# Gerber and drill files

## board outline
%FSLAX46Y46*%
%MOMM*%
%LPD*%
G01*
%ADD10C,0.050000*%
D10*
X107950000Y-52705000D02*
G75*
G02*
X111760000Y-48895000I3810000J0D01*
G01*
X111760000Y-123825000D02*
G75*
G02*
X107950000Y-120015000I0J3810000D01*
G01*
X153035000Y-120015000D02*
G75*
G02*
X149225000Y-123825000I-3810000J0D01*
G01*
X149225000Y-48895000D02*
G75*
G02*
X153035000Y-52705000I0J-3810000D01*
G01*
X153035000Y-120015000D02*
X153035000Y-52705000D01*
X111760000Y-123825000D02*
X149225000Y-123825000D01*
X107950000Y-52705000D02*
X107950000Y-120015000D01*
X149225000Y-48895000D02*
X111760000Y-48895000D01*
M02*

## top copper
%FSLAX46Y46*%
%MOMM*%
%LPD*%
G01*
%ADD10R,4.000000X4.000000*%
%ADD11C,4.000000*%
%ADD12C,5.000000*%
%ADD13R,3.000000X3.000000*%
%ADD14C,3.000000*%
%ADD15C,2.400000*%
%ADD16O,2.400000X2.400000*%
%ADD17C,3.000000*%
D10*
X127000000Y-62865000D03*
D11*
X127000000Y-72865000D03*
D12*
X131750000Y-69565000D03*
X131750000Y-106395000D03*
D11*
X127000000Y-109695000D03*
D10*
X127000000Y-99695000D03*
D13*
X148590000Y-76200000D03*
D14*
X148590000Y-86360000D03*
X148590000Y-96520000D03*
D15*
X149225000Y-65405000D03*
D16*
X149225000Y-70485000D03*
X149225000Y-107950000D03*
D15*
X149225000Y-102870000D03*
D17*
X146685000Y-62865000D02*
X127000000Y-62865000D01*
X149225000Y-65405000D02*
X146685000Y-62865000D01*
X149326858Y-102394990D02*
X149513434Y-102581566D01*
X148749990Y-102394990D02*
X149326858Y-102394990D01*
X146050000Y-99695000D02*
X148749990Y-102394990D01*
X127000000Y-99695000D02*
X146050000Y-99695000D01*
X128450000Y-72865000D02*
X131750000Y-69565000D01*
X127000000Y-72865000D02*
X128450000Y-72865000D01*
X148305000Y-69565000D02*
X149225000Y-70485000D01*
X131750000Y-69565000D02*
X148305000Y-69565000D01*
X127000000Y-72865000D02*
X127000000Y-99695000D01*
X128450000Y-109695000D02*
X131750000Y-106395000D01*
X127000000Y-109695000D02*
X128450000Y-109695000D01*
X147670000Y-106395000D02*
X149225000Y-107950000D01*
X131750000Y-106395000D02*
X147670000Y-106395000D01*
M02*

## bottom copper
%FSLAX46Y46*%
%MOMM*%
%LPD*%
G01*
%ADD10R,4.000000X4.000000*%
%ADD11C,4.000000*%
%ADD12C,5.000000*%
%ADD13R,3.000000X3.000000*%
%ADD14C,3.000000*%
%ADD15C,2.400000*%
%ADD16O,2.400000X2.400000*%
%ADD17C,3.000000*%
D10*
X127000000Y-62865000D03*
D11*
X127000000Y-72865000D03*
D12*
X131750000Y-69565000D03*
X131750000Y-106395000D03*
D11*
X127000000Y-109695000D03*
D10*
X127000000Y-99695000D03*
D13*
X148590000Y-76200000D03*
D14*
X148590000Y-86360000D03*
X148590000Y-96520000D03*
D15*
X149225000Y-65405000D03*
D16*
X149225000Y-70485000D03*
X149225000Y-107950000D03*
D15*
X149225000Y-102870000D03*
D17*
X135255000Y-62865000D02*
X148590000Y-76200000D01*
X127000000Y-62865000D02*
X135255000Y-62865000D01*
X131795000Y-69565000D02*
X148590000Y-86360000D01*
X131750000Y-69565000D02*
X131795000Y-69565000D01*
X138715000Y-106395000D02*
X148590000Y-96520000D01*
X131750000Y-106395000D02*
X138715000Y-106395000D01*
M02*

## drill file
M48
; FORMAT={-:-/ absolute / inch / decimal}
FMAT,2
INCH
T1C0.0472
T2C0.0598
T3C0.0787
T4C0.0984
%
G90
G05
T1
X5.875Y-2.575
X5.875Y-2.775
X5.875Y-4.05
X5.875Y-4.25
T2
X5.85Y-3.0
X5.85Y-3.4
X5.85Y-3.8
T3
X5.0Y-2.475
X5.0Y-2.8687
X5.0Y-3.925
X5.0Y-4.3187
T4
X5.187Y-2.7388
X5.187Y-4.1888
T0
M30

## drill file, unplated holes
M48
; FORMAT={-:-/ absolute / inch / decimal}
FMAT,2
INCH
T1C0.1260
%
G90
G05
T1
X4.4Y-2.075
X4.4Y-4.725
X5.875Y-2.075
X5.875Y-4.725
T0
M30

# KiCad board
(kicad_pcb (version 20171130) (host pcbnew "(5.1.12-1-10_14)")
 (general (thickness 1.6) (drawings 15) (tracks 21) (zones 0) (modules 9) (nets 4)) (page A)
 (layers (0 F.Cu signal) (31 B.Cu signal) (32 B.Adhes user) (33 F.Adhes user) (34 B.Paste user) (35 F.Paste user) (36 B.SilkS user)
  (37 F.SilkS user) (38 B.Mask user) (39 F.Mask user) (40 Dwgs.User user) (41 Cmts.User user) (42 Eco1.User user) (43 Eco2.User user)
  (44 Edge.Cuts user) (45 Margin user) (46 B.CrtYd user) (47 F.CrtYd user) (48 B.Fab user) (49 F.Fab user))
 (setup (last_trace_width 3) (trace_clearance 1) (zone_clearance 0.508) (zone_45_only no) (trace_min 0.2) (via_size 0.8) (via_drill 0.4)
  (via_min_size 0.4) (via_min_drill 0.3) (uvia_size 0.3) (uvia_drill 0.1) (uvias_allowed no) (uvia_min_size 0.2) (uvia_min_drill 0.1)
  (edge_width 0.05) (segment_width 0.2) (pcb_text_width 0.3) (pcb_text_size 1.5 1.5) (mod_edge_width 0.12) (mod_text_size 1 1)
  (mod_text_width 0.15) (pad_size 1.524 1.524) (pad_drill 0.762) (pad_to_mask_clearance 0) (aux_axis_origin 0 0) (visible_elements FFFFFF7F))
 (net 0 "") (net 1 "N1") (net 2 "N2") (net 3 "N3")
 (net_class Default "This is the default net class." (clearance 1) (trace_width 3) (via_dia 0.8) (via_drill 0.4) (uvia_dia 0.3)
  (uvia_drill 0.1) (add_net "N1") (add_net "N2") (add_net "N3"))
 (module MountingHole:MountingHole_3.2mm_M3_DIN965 (layer F.Cu) (at 111.76 52.705)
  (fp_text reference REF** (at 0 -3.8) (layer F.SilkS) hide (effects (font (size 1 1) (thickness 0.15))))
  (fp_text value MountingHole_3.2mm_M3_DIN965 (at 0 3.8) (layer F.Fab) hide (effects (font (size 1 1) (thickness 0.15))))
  (pad 1 np_thru_hole circle (at 0 0) (size 3.2 3.2) (drill 3.2) (layers *.Cu *.Mask)))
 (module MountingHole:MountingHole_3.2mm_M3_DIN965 (layer F.Cu) (at 111.76 120.015)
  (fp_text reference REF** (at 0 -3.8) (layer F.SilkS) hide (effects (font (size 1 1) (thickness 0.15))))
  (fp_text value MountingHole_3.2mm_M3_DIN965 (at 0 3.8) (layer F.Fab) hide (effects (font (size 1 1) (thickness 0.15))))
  (pad 1 np_thru_hole circle (at 0 0) (size 3.2 3.2) (drill 3.2) (layers *.Cu *.Mask)))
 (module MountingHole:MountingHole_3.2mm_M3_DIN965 (layer F.Cu) (at 149.225 120.015)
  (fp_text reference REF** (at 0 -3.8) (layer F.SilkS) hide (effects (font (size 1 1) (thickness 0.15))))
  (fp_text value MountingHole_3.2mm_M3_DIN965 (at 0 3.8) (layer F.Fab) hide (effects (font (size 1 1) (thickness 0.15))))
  (pad 1 np_thru_hole circle (at 0 0) (size 3.2 3.2) (drill 3.2) (layers *.Cu *.Mask)))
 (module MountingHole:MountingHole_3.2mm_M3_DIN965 (layer F.Cu) (at 149.225 52.705)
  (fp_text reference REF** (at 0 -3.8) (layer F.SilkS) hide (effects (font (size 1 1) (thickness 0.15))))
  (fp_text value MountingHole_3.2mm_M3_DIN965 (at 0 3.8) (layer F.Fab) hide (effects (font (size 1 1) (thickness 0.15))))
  (pad 1 np_thru_hole circle (at 0 0) (size 3.2 3.2) (drill 3.2) (layers *.Cu *.Mask)))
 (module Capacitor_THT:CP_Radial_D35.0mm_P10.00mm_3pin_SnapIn (layer F.Cu) (at 127 62.865 270)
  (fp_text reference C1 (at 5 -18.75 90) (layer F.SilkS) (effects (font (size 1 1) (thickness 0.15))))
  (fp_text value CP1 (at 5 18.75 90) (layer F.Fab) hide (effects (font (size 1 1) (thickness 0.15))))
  (pad 1 thru_hole rect (at 0 0 270) (size 4 4) (drill 2) (layers *.Cu *.Mask) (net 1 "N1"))
  (pad 2 thru_hole circle (at 10 0 270) (size 4 4) (drill 2) (layers *.Cu *.Mask) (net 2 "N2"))
  (pad 2 thru_hole circle (at 6.7 -4.75 270) (size 5 5) (drill 2.5) (layers *.Cu *.Mask) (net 2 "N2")))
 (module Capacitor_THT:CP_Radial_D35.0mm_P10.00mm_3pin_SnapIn (layer F.Cu) (at 127 99.695 270)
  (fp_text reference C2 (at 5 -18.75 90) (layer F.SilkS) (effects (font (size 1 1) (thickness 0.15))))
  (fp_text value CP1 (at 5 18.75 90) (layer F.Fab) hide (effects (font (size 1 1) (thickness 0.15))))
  (pad 2 thru_hole circle (at 6.7 -4.75 270) (size 5 5) (drill 2.5) (layers *.Cu *.Mask) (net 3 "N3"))
  (pad 2 thru_hole circle (at 10 0 270) (size 4 4) (drill 2) (layers *.Cu *.Mask) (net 3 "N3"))
  (pad 1 thru_hole rect (at 0 0 270) (size 4 4) (drill 2) (layers *.Cu *.Mask) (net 2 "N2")))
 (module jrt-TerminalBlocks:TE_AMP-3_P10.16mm (layer F.Cu) (at 148.59 76.2 270)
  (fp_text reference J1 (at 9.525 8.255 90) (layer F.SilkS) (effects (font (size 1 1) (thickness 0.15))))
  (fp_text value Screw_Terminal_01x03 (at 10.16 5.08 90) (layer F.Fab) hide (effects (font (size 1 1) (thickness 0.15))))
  (pad 1 thru_hole rect (at 0 0 270) (size 3 3) (drill 1.52) (layers *.Cu *.Mask) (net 1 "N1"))
  (pad 2 thru_hole circle (at 10.16 0 270) (size 3 3) (drill 1.52) (layers *.Cu *.Mask) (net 2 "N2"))
  (pad 3 thru_hole circle (at 20.32 0 270) (size 3 3) (drill 1.52) (layers *.Cu *.Mask) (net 3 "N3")))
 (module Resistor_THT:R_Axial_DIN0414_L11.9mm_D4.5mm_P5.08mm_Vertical (layer F.Cu) (at 149.225 65.405 270)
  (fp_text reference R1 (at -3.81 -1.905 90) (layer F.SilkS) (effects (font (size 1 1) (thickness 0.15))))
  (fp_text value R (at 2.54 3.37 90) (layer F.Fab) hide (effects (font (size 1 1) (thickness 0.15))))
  (pad 1 thru_hole circle (at 0 0 270) (size 2.4 2.4) (drill 1.2) (layers *.Cu *.Mask) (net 1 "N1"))
  (pad 2 thru_hole oval (at 5.08 0 270) (size 2.4 2.4) (drill 1.2) (layers *.Cu *.Mask) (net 2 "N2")))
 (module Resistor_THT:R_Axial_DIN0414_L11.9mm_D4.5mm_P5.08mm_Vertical (layer F.Cu) (at 149.225 102.87 270)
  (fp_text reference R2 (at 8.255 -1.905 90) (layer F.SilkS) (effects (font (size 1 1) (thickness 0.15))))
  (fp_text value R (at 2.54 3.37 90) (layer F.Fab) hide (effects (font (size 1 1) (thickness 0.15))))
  (pad 2 thru_hole oval (at 5.08 0 270) (size 2.4 2.4) (drill 1.2) (layers *.Cu *.Mask) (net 3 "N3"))
  (pad 1 thru_hole circle (at 0 0 270) (size 2.4 2.4) (drill 1.2) (layers *.Cu *.Mask) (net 2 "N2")))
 (gr_arc (start 111.76 52.705) (end 111.76 48.895) (angle -90) (layer Edge.Cuts) (width 0.05))
 (gr_arc (start 111.76 120.015) (end 107.95 120.015) (angle -90) (layer Edge.Cuts) (width 0.05))
 (gr_arc (start 149.225 120.015) (end 149.225 123.825) (angle -90) (layer Edge.Cuts) (width 0.05))
 (gr_arc (start 149.225 52.705) (end 153.035 52.705) (angle -90) (layer Edge.Cuts) (width 0.05))
 (gr_line (start 153.035 120.015) (end 153.035 52.705) (layer Edge.Cuts) (width 0.05))
 (gr_line (start 111.76 123.825) (end 149.225 123.825) (layer Edge.Cuts) (width 0.05))
 (gr_line (start 107.95 52.705) (end 107.95 120.015) (layer Edge.Cuts) (width 0.05))
 (gr_line (start 149.225 48.895) (end 111.76 48.895) (layer Edge.Cuts) (width 0.05))
 (segment (start 146.685 62.865) (end 127 62.865) (width 3) (layer F.Cu) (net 1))
 (segment (start 149.225 65.405) (end 146.685 62.865) (width 3) (layer F.Cu) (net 1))
 (segment (start 135.255 62.865) (end 148.59 76.2) (width 3) (layer B.Cu) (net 1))
 (segment (start 127 62.865) (end 135.255 62.865) (width 3) (layer B.Cu) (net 1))
 (segment (start 149.326858 102.39499) (end 149.513434 102.581566) (width 3) (layer F.Cu) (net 2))
 (segment (start 148.74999 102.39499) (end 149.326858 102.39499) (width 3) (layer F.Cu) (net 2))
 (segment (start 146.05 99.695) (end 148.74999 102.39499) (width 3) (layer F.Cu) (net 2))
 (segment (start 127 99.695) (end 146.05 99.695) (width 3) (layer F.Cu) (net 2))
 (segment (start 128.45 72.865) (end 131.75 69.565) (width 3) (layer F.Cu) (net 2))
 (segment (start 127 72.865) (end 128.45 72.865) (width 3) (layer F.Cu) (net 2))
 (segment (start 148.305 69.565) (end 149.225 70.485) (width 3) (layer F.Cu) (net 2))
 (segment (start 131.75 69.565) (end 148.305 69.565) (width 3) (layer F.Cu) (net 2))
 (segment (start 127 72.865) (end 127 99.695) (width 3) (layer F.Cu) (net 2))
 (segment (start 131.795 69.565) (end 148.59 86.36) (width 3) (layer B.Cu) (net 2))
 (segment (start 131.75 69.565) (end 131.795 69.565) (width 3) (layer B.Cu) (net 2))
 (segment (start 128.45 109.695) (end 131.75 106.395) (width 3) (layer F.Cu) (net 3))
 (segment (start 127 109.695) (end 128.45 109.695) (width 3) (layer F.Cu) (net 3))
 (segment (start 147.67 106.395) (end 149.225 107.95) (width 3) (layer F.Cu) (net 3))
 (segment (start 131.75 106.395) (end 147.67 106.395) (width 3) (layer F.Cu) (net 3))
 (segment (start 138.715 106.395) (end 148.59 96.52) (width 3) (layer B.Cu) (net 3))
 (segment (start 131.75 106.395) (end 138.715 106.395) (width 3) (layer B.Cu) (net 3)))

